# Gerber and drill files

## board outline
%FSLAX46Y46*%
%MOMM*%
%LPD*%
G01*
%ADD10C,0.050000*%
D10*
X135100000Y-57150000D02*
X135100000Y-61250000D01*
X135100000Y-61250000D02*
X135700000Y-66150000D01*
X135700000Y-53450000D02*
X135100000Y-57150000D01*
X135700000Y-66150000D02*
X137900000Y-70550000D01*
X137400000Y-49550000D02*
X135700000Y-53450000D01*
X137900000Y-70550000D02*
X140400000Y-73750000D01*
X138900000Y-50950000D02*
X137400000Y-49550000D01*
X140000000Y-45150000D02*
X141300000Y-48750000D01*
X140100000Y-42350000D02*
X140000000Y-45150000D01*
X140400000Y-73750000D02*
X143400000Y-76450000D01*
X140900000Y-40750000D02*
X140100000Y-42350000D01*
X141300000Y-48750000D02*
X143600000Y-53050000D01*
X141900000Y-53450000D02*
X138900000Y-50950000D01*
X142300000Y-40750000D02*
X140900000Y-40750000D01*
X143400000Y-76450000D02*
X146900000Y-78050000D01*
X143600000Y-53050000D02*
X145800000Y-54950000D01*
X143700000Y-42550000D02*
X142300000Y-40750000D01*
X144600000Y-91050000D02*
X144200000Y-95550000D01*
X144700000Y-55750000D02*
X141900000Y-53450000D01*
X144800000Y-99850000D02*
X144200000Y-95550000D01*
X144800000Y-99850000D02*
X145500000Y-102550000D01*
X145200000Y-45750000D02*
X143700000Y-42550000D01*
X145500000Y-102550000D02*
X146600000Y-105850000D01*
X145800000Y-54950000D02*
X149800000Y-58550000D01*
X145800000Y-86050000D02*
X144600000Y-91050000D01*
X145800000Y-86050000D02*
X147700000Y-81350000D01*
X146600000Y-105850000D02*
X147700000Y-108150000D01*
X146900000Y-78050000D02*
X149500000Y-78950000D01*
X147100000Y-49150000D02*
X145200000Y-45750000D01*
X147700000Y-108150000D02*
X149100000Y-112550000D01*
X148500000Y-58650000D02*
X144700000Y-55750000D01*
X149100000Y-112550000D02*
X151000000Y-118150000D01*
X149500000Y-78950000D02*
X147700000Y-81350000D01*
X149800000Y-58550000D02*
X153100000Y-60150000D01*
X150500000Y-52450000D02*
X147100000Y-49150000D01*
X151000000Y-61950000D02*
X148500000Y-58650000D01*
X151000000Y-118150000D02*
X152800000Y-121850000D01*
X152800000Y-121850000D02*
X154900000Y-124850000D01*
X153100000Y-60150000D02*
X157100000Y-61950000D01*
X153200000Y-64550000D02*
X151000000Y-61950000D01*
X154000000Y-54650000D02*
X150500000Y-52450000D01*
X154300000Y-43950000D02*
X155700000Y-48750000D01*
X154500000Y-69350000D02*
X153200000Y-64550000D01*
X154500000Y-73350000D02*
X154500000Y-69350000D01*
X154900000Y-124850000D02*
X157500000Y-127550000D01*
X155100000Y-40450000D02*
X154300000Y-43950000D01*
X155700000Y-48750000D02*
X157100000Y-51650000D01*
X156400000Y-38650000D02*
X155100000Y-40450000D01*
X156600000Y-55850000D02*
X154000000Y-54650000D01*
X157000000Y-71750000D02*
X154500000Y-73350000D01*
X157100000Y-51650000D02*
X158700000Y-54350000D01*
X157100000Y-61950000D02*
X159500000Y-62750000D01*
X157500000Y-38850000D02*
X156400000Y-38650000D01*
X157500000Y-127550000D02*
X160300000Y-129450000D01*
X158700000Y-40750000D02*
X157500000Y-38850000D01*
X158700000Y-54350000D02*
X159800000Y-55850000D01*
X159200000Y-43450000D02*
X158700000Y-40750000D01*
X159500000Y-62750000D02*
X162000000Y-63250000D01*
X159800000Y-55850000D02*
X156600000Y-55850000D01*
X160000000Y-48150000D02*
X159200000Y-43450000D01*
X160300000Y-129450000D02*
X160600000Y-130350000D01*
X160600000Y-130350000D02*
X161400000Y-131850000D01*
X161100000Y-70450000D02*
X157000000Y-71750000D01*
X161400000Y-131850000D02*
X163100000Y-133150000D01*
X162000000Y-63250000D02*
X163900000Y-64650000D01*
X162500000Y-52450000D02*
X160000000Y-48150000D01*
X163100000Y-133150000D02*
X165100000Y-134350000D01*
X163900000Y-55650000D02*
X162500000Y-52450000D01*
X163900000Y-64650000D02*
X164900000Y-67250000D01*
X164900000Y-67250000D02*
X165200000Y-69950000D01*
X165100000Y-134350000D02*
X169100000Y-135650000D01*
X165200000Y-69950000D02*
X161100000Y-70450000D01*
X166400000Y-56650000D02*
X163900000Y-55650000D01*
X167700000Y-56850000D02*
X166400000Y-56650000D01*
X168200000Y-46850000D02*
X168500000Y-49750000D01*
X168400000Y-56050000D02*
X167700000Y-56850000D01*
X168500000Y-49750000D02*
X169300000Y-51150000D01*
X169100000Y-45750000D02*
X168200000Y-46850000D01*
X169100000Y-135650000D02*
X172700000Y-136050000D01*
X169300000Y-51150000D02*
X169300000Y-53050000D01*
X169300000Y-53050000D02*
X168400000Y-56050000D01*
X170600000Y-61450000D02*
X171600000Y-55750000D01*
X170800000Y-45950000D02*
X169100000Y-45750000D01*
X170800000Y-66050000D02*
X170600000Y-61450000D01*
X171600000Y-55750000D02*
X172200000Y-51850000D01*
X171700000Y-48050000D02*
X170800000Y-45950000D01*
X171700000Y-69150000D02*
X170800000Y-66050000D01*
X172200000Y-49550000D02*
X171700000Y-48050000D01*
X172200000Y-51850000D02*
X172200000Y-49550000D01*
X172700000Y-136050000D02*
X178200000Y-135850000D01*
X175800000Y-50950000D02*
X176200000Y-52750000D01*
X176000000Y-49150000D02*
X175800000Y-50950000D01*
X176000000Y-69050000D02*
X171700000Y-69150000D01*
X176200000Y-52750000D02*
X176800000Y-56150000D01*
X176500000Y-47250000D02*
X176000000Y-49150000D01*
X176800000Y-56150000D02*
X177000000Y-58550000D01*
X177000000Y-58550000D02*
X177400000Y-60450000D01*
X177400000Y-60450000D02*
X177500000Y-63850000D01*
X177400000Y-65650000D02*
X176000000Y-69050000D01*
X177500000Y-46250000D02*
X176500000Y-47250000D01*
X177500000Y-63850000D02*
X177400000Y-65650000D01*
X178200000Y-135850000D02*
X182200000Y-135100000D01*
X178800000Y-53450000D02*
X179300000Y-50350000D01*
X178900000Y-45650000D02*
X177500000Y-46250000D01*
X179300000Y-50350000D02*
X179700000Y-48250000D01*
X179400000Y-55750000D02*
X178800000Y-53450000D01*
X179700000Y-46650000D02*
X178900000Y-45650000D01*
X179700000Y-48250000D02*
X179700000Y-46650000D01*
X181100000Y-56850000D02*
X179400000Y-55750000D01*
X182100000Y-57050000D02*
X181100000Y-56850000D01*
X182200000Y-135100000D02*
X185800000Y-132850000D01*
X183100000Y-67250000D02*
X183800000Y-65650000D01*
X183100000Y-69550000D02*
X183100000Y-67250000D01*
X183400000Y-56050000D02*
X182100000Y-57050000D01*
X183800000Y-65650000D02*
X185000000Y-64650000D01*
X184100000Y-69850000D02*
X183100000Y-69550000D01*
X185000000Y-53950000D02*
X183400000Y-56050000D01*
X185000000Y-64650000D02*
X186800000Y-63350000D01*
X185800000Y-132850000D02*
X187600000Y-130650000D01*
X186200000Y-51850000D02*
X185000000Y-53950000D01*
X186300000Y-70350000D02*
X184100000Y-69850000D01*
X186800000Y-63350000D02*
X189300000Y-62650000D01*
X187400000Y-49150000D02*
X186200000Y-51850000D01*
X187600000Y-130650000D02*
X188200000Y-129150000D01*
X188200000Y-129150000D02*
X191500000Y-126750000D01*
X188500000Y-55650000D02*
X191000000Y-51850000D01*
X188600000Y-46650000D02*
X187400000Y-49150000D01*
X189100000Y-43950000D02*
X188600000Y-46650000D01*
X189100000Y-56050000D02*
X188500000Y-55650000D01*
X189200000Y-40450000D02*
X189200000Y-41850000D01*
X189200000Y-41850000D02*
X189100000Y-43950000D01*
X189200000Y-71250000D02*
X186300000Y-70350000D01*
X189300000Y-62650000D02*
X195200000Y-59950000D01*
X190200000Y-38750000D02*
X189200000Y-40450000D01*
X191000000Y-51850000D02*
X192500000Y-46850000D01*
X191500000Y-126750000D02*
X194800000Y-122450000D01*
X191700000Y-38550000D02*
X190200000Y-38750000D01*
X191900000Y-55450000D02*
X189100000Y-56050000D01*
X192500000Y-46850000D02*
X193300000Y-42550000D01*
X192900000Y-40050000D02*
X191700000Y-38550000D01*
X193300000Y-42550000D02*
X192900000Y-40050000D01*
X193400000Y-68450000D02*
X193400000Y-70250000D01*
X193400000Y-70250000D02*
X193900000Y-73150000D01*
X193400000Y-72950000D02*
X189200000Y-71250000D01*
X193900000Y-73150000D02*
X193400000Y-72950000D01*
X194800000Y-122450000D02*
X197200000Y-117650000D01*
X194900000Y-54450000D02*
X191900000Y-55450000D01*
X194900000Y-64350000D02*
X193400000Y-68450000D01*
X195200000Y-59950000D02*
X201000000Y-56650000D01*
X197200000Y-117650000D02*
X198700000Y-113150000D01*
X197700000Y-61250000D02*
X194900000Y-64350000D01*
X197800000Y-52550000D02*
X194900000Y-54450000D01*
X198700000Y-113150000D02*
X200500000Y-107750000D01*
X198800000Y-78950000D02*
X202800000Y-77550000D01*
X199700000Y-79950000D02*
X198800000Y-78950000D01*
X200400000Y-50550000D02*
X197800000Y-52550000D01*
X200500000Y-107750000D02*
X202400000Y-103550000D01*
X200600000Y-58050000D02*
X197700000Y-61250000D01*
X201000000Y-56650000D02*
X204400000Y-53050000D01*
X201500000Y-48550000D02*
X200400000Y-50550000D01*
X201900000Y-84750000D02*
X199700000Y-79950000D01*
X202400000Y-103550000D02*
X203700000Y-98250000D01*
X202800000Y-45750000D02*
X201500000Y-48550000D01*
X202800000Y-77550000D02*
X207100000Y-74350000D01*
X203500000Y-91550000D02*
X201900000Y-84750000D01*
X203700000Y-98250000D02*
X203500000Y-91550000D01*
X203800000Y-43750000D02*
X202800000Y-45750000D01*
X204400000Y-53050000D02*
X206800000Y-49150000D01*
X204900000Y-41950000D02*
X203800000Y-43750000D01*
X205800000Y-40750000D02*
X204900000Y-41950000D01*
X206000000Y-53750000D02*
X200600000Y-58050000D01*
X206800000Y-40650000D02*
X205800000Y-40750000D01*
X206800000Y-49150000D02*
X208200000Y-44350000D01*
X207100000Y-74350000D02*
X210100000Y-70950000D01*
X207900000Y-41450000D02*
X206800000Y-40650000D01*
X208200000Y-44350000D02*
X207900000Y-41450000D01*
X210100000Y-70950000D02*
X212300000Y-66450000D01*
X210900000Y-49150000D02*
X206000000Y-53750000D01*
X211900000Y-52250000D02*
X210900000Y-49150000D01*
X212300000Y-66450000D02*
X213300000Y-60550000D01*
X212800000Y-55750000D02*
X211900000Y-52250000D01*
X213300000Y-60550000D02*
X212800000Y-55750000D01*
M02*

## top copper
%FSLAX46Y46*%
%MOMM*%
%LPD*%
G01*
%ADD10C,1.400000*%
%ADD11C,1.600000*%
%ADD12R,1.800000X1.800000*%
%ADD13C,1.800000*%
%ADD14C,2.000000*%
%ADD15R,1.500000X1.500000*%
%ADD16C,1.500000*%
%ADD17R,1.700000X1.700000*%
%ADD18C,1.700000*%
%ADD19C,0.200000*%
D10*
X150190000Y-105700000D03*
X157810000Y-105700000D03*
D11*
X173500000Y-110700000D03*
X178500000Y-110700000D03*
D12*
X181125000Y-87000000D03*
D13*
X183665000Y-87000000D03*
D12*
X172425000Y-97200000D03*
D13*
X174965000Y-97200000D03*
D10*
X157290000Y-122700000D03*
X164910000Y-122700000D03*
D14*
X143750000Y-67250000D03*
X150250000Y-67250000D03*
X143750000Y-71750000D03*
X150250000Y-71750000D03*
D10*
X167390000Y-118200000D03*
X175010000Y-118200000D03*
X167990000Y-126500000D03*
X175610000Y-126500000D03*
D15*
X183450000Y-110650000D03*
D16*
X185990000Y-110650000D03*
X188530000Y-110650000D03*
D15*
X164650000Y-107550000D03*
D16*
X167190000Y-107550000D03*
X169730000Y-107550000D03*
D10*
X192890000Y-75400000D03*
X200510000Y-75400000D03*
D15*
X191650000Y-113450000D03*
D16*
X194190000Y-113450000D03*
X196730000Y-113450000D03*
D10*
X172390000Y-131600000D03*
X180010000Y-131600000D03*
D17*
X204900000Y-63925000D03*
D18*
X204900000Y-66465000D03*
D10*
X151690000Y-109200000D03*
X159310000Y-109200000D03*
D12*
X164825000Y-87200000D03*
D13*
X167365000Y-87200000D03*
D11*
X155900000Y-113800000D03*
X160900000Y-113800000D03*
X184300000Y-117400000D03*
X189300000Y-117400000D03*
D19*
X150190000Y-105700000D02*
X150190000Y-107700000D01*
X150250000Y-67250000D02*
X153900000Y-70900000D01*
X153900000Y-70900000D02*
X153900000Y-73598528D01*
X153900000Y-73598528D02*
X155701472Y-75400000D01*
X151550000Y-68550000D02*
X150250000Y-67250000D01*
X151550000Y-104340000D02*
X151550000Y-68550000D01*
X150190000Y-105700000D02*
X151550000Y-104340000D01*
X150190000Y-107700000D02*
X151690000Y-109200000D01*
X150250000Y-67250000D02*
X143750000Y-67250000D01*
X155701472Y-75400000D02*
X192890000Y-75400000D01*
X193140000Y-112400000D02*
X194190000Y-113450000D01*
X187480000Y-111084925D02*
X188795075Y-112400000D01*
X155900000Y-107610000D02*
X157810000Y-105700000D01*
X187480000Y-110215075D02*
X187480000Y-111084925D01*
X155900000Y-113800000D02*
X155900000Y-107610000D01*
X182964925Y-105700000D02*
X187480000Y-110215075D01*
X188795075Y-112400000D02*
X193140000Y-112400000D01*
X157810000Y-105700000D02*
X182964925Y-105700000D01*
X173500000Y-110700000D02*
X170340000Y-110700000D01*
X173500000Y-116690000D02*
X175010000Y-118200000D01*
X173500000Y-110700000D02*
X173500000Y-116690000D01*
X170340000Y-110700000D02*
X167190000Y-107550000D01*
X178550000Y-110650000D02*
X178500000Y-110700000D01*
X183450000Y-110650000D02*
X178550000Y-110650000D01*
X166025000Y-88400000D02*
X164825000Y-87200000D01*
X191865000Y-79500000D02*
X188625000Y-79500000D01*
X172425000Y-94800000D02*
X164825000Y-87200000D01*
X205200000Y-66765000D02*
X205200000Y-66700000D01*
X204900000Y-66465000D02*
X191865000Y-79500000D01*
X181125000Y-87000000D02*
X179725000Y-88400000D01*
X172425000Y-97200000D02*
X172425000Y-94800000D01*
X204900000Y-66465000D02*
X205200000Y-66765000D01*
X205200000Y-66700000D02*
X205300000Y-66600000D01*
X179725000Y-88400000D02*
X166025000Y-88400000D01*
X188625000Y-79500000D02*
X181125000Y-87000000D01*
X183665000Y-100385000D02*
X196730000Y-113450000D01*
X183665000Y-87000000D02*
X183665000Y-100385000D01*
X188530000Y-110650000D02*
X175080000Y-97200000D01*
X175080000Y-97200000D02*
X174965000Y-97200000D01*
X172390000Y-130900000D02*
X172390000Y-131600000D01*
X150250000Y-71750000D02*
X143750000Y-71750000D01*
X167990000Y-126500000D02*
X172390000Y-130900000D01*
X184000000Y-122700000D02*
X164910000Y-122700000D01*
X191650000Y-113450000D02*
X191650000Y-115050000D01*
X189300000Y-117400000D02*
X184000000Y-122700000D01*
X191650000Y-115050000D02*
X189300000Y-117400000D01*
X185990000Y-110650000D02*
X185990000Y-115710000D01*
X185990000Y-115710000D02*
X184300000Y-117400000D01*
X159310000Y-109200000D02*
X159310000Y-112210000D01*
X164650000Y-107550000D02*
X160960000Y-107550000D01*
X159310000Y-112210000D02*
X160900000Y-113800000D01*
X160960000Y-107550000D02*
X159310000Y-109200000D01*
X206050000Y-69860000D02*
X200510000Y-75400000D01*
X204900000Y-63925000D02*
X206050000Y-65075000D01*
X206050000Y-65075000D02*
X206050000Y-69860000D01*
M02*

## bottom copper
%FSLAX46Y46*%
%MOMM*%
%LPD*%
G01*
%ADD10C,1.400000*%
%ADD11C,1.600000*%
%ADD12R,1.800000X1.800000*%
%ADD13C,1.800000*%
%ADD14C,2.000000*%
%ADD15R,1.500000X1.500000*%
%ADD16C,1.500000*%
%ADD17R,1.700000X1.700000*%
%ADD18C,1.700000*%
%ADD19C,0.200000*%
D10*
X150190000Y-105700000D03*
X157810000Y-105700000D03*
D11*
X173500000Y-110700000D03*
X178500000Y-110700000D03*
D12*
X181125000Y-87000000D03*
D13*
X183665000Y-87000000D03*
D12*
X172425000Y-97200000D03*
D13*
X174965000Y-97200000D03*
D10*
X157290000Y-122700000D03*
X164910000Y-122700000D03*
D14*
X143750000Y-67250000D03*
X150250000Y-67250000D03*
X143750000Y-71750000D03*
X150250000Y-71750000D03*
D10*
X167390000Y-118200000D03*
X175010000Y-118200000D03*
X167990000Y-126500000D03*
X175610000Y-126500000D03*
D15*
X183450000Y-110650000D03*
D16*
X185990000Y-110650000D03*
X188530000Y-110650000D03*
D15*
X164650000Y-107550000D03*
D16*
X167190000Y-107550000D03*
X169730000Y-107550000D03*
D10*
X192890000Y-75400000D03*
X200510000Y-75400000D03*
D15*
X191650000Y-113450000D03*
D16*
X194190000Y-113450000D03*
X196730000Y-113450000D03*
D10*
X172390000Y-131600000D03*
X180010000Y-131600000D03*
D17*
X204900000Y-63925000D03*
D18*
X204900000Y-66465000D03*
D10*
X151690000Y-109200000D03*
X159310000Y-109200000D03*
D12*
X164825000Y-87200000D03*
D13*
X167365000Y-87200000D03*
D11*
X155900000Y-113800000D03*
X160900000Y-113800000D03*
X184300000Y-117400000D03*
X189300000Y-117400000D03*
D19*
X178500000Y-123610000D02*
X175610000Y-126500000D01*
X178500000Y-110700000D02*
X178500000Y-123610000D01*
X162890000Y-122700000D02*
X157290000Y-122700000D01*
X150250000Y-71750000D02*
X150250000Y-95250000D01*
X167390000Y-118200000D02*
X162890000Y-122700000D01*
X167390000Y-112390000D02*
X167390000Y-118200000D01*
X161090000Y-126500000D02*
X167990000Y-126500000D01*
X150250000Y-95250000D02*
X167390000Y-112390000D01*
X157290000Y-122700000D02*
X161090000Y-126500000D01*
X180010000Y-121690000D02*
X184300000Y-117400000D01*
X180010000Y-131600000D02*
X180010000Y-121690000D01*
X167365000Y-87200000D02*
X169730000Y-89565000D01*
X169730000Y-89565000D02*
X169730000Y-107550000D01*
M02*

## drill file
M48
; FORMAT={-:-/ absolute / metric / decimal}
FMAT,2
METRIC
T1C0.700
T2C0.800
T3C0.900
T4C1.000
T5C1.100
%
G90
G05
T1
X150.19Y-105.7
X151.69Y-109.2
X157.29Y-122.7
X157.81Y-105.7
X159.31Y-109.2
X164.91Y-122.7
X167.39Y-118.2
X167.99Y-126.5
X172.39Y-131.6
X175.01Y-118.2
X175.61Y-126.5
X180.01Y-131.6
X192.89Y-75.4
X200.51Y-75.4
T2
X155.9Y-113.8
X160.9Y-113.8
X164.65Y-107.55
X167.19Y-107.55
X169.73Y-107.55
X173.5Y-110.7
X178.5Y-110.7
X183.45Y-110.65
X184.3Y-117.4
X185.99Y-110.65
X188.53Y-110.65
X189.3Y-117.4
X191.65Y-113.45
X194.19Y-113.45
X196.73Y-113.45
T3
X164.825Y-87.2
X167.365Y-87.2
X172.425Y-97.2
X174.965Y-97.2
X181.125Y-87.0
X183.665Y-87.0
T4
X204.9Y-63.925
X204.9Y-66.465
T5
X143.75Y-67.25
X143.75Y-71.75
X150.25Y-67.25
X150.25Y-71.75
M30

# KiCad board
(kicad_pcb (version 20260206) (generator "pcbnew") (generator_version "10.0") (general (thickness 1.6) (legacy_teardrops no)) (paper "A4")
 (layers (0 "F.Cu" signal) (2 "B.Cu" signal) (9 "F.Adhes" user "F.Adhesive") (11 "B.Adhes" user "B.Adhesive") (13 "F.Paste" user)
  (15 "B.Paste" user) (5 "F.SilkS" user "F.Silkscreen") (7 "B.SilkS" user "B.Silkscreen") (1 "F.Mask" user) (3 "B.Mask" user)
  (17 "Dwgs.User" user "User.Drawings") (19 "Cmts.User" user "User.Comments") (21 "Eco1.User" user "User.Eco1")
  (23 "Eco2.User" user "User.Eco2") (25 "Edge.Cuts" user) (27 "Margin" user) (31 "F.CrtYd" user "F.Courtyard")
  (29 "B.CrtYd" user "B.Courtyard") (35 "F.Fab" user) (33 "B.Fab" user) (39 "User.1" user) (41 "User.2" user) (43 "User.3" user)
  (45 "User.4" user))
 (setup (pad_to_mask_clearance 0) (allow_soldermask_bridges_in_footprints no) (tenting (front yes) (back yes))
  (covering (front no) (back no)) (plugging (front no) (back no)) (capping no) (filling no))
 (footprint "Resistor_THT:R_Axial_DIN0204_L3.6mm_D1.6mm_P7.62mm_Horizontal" (layer "F.Cu") (at 150.19 105.7)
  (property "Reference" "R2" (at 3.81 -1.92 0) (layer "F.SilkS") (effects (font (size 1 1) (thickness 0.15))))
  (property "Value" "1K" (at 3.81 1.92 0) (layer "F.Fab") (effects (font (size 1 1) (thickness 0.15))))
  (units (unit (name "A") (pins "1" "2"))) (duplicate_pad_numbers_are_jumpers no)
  (pad "1" thru_hole circle (at 0 0) (size 1.4 1.4) (drill 0.7) (layers "*.Cu" "*.Mask") (remove_unused_layers no) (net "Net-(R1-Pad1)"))
  (pad "2" thru_hole circle (at 7.62 0) (size 1.4 1.4) (drill 0.7) (layers "*.Cu" "*.Mask") (remove_unused_layers no) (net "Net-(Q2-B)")))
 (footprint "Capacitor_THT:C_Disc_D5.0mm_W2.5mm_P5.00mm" (layer "F.Cu") (at 173.5 110.7)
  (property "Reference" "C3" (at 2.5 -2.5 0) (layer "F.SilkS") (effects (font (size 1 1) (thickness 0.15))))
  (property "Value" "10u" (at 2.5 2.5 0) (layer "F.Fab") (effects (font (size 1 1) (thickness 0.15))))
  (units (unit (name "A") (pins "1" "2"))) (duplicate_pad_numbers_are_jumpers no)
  (pad "1" thru_hole circle (at 0 0) (size 1.6 1.6) (drill 0.8) (layers "*.Cu" "*.Mask") (remove_unused_layers no) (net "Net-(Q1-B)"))
  (pad "2" thru_hole circle (at 5 0) (size 1.6 1.6) (drill 0.8) (layers "*.Cu" "*.Mask") (remove_unused_layers no) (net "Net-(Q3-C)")))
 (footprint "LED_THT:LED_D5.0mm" (layer "F.Cu") (at 181.125 87)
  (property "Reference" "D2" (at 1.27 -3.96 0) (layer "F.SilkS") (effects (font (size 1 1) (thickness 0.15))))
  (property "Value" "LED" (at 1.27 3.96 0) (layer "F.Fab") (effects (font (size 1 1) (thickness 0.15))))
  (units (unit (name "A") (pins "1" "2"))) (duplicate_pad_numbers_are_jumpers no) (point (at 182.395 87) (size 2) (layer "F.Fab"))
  (pad "1" thru_hole rect (at 0 0) (size 1.8 1.8) (drill 0.9) (layers "*.Cu" "*.Mask") (remove_unused_layers no) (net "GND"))
  (pad "2" thru_hole circle (at 2.54 0) (size 1.8 1.8) (drill 0.9) (layers "*.Cu" "*.Mask") (remove_unused_layers no) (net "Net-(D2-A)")))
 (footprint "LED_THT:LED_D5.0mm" (layer "F.Cu") (at 172.425 97.2)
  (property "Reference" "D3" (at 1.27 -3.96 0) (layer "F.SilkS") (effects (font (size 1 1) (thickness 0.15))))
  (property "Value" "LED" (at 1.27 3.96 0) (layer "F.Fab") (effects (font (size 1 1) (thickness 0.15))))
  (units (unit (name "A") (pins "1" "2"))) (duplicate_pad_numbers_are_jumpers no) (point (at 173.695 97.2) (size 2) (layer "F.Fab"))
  (pad "1" thru_hole rect (at 0 0) (size 1.8 1.8) (drill 0.9) (layers "*.Cu" "*.Mask") (remove_unused_layers no) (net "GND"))
  (pad "2" thru_hole circle (at 2.54 0) (size 1.8 1.8) (drill 0.9) (layers "*.Cu" "*.Mask") (remove_unused_layers no) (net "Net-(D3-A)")))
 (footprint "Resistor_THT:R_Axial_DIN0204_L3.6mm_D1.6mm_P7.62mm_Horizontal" (layer "F.Cu") (at 157.29 122.7)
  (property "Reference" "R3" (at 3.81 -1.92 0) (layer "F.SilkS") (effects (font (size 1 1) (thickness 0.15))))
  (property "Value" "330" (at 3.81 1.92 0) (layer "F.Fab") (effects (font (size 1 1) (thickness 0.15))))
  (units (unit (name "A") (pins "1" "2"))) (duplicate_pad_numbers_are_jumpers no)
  (pad "1" thru_hole circle (at 0 0) (size 1.4 1.4) (drill 0.7) (layers "*.Cu" "*.Mask") (remove_unused_layers no) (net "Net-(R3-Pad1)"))
  (pad "2" thru_hole circle (at 7.62 0) (size 1.4 1.4) (drill 0.7) (layers "*.Cu" "*.Mask") (remove_unused_layers no) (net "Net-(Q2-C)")))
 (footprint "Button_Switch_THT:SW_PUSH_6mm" (layer "F.Cu") (at 143.75 67.25)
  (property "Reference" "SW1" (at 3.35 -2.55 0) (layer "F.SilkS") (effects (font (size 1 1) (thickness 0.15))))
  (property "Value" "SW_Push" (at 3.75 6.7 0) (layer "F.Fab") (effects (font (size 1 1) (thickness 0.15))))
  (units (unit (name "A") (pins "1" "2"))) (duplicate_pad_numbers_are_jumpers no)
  (pad "1" thru_hole circle (at 0 0 90) (size 2 2) (drill 1.1) (layers "*.Cu" "*.Mask") (remove_unused_layers no) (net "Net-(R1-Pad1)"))
  (pad "1" thru_hole circle (at 6.5 0 90) (size 2 2) (drill 1.1) (layers "*.Cu" "*.Mask") (remove_unused_layers no) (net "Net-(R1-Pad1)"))
  (pad "2" thru_hole circle (at 0 4.5 90) (size 2 2) (drill 1.1) (layers "*.Cu" "*.Mask") (remove_unused_layers no) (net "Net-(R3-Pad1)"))
  (pad "2" thru_hole circle (at 6.5 4.5 90) (size 2 2) (drill 1.1) (layers "*.Cu" "*.Mask") (remove_unused_layers no) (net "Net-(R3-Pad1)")))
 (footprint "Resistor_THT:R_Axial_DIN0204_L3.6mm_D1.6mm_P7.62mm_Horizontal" (layer "F.Cu") (at 167.39 118.2)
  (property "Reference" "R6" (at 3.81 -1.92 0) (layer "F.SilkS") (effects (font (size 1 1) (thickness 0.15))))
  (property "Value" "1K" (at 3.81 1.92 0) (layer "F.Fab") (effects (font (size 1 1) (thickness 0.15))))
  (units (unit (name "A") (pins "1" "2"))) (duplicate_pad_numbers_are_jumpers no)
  (pad "1" thru_hole circle (at 0 0) (size 1.4 1.4) (drill 0.7) (layers "*.Cu" "*.Mask") (remove_unused_layers no) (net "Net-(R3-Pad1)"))
  (pad "2" thru_hole circle (at 7.62 0) (size 1.4 1.4) (drill 0.7) (layers "*.Cu" "*.Mask") (remove_unused_layers no) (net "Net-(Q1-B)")))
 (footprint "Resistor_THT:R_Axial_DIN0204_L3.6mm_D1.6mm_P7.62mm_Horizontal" (layer "F.Cu") (at 167.99 126.5)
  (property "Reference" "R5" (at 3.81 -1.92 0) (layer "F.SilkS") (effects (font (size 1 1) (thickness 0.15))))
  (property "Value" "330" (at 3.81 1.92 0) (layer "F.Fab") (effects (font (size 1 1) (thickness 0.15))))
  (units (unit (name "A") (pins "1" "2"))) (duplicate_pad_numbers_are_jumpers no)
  (pad "1" thru_hole circle (at 0 0) (size 1.4 1.4) (drill 0.7) (layers "*.Cu" "*.Mask") (remove_unused_layers no) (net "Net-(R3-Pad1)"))
  (pad "2" thru_hole circle (at 7.62 0) (size 1.4 1.4) (drill 0.7) (layers "*.Cu" "*.Mask") (remove_unused_layers no) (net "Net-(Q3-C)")))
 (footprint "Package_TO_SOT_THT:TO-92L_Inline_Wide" (layer "F.Cu") (at 183.45 110.65)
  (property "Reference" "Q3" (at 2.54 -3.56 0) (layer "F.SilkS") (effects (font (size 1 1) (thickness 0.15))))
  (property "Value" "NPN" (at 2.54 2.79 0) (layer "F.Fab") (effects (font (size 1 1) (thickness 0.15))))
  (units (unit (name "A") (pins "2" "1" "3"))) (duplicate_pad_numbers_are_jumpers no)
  (pad "1" thru_hole rect (at 0 0) (size 1.5 1.5) (drill 0.8) (layers "*.Cu" "*.Mask") (remove_unused_layers no) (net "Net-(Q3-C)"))
  (pad "2" thru_hole circle (at 2.54 0) (size 1.5 1.5) (drill 0.8) (layers "*.Cu" "*.Mask") (remove_unused_layers no) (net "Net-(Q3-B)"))
  (pad "3" thru_hole circle (at 5.08 0) (size 1.5 1.5) (drill 0.8) (layers "*.Cu" "*.Mask") (remove_unused_layers no) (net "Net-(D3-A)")))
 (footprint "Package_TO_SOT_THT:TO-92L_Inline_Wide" (layer "F.Cu") (at 164.65 107.55)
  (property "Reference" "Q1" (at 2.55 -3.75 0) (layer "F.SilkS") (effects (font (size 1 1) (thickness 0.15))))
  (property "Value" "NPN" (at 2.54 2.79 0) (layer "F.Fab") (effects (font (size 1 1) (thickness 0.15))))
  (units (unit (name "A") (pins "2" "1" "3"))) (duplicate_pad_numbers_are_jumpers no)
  (pad "1" thru_hole rect (at 0 0) (size 1.5 1.5) (drill 0.8) (layers "*.Cu" "*.Mask") (remove_unused_layers no) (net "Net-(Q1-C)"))
  (pad "2" thru_hole circle (at 2.54 0) (size 1.5 1.5) (drill 0.8) (layers "*.Cu" "*.Mask") (remove_unused_layers no) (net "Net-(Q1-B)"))
  (pad "3" thru_hole circle (at 5.08 0) (size 1.5 1.5) (drill 0.8) (layers "*.Cu" "*.Mask") (remove_unused_layers no) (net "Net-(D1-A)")))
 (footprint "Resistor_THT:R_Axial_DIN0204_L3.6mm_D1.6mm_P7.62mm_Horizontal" (layer "F.Cu") (at 192.89 75.4)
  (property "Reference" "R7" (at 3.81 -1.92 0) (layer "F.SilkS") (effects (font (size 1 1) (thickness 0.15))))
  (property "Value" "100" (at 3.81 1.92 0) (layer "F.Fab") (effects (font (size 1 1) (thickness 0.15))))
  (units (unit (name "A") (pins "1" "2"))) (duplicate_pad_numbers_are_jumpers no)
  (pad "1" thru_hole circle (at 0 0) (size 1.4 1.4) (drill 0.7) (layers "*.Cu" "*.Mask") (remove_unused_layers no) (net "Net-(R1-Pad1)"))
  (pad "2" thru_hole circle (at 7.62 0) (size 1.4 1.4) (drill 0.7) (layers "*.Cu" "*.Mask") (remove_unused_layers no) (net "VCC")))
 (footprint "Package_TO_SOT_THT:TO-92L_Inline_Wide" (layer "F.Cu") (at 191.65 113.45)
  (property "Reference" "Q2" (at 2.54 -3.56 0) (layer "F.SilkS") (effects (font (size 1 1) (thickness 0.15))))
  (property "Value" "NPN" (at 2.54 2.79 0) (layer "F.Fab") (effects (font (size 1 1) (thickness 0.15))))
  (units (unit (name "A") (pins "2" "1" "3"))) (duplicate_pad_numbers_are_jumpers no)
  (pad "1" thru_hole rect (at 0 0) (size 1.5 1.5) (drill 0.8) (layers "*.Cu" "*.Mask") (remove_unused_layers no) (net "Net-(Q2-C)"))
  (pad "2" thru_hole circle (at 2.54 0) (size 1.5 1.5) (drill 0.8) (layers "*.Cu" "*.Mask") (remove_unused_layers no) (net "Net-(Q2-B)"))
  (pad "3" thru_hole circle (at 5.08 0) (size 1.5 1.5) (drill 0.8) (layers "*.Cu" "*.Mask") (remove_unused_layers no) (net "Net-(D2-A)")))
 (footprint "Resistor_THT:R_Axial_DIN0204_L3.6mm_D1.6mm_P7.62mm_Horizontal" (layer "F.Cu") (at 172.39 131.6)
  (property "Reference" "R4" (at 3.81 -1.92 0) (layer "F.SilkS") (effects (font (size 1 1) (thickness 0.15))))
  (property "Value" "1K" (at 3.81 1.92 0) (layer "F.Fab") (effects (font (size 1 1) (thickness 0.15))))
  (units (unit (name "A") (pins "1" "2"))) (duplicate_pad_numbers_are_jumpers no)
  (pad "1" thru_hole circle (at 0 0) (size 1.4 1.4) (drill 0.7) (layers "*.Cu" "*.Mask") (remove_unused_layers no) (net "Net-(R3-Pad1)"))
  (pad "2" thru_hole circle (at 7.62 0) (size 1.4 1.4) (drill 0.7) (layers "*.Cu" "*.Mask") (remove_unused_layers no) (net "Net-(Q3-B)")))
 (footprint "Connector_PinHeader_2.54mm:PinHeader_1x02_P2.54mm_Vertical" (layer "F.Cu") (at 204.9 63.925)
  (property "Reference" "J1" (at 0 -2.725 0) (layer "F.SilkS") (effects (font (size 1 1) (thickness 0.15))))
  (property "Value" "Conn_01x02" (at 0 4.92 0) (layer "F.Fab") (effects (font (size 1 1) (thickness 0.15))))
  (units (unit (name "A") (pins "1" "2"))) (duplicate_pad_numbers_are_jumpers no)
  (pad "1" thru_hole rect (at 0 0) (size 1.7 1.7) (drill 1) (layers "*.Cu" "*.Mask") (remove_unused_layers no) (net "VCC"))
  (pad "2" thru_hole circle (at 0 2.54) (size 1.7 1.7) (drill 1) (layers "*.Cu" "*.Mask") (remove_unused_layers no) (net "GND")))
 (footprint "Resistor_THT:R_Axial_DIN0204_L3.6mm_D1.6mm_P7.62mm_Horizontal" (layer "F.Cu") (at 151.69 109.2)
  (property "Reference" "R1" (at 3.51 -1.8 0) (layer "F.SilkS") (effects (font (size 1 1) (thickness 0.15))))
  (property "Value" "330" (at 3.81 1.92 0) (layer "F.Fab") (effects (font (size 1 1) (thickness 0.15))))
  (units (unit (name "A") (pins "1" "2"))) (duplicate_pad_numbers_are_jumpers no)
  (pad "1" thru_hole circle (at 0 0) (size 1.4 1.4) (drill 0.7) (layers "*.Cu" "*.Mask") (remove_unused_layers no) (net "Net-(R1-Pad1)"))
  (pad "2" thru_hole circle (at 7.62 0) (size 1.4 1.4) (drill 0.7) (layers "*.Cu" "*.Mask") (remove_unused_layers no) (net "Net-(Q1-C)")))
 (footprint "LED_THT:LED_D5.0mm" (layer "F.Cu") (at 164.825 87.2)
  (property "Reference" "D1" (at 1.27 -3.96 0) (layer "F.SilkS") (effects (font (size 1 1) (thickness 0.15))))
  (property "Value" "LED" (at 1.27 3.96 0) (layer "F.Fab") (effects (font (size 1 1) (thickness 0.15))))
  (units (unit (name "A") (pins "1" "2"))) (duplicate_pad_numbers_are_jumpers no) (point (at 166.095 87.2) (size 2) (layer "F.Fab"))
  (pad "1" thru_hole rect (at 0 0) (size 1.8 1.8) (drill 0.9) (layers "*.Cu" "*.Mask") (remove_unused_layers no) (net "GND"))
  (pad "2" thru_hole circle (at 2.54 0) (size 1.8 1.8) (drill 0.9) (layers "*.Cu" "*.Mask") (remove_unused_layers no) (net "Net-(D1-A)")))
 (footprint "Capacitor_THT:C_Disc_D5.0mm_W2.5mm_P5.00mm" (layer "F.Cu") (at 155.9 113.8)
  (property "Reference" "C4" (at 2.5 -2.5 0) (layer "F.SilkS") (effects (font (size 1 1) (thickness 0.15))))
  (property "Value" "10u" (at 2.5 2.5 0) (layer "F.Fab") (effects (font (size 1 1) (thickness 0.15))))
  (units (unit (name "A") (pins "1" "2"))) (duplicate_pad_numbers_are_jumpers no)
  (pad "1" thru_hole circle (at 0 0) (size 1.6 1.6) (drill 0.8) (layers "*.Cu" "*.Mask") (remove_unused_layers no) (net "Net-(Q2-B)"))
  (pad "2" thru_hole circle (at 5 0) (size 1.6 1.6) (drill 0.8) (layers "*.Cu" "*.Mask") (remove_unused_layers no) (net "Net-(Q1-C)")))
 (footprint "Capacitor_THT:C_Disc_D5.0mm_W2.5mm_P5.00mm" (layer "F.Cu") (at 184.3 117.4)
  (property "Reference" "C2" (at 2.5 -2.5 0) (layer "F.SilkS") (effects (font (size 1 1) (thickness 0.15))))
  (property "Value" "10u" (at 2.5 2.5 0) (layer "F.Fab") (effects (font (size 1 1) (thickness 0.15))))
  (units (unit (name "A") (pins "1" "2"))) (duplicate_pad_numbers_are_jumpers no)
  (pad "1" thru_hole circle (at 0 0) (size 1.6 1.6) (drill 0.8) (layers "*.Cu" "*.Mask") (remove_unused_layers no) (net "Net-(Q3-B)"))
  (pad "2" thru_hole circle (at 5 0) (size 1.6 1.6) (drill 0.8) (layers "*.Cu" "*.Mask") (remove_unused_layers no) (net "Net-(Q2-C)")))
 (gr_line (start 135.1 57.15) (end 135.1 61.25) (stroke (width 0.05) (type default)) (layer "Edge.Cuts"))
 (gr_line (start 135.1 61.25) (end 135.7 66.15) (stroke (width 0.05) (type default)) (layer "Edge.Cuts"))
 (gr_line (start 135.7 53.45) (end 135.1 57.15) (stroke (width 0.05) (type default)) (layer "Edge.Cuts"))
 (gr_line (start 135.7 66.15) (end 137.9 70.55) (stroke (width 0.05) (type default)) (layer "Edge.Cuts"))
 (gr_line (start 137.4 49.55) (end 135.7 53.45) (stroke (width 0.05) (type default)) (layer "Edge.Cuts"))
 (gr_line (start 137.9 70.55) (end 140.4 73.75) (stroke (width 0.05) (type default)) (layer "Edge.Cuts"))
 (gr_line (start 138.9 50.95) (end 137.4 49.55) (stroke (width 0.05) (type default)) (layer "Edge.Cuts"))
 (gr_line (start 140 45.15) (end 141.3 48.75) (stroke (width 0.05) (type default)) (layer "Edge.Cuts"))
 (gr_line (start 140.1 42.35) (end 140 45.15) (stroke (width 0.05) (type default)) (layer "Edge.Cuts"))
 (gr_line (start 140.4 73.75) (end 143.4 76.45) (stroke (width 0.05) (type default)) (layer "Edge.Cuts"))
 (gr_line (start 140.9 40.75) (end 140.1 42.35) (stroke (width 0.05) (type default)) (layer "Edge.Cuts"))
 (gr_line (start 141.3 48.75) (end 143.6 53.05) (stroke (width 0.05) (type default)) (layer "Edge.Cuts"))
 (gr_line (start 141.9 53.45) (end 138.9 50.95) (stroke (width 0.05) (type default)) (layer "Edge.Cuts"))
 (gr_line (start 142.3 40.75) (end 140.9 40.75) (stroke (width 0.05) (type default)) (layer "Edge.Cuts"))
 (gr_line (start 143.4 76.45) (end 146.9 78.05) (stroke (width 0.05) (type default)) (layer "Edge.Cuts"))
 (gr_line (start 143.6 53.05) (end 145.8 54.95) (stroke (width 0.05) (type default)) (layer "Edge.Cuts"))
 (gr_line (start 143.7 42.55) (end 142.3 40.75) (stroke (width 0.05) (type default)) (layer "Edge.Cuts"))
 (gr_line (start 144.6 91.05) (end 144.2 95.55) (stroke (width 0.05) (type default)) (layer "Edge.Cuts"))
 (gr_line (start 144.7 55.75) (end 141.9 53.45) (stroke (width 0.05) (type default)) (layer "Edge.Cuts"))
 (gr_line (start 144.8 99.85) (end 144.2 95.55) (stroke (width 0.05) (type default)) (layer "Edge.Cuts"))
 (gr_line (start 144.8 99.85) (end 145.5 102.55) (stroke (width 0.05) (type default)) (layer "Edge.Cuts"))
 (gr_line (start 145.2 45.75) (end 143.7 42.55) (stroke (width 0.05) (type default)) (layer "Edge.Cuts"))
 (gr_line (start 145.5 102.55) (end 146.6 105.85) (stroke (width 0.05) (type default)) (layer "Edge.Cuts"))
 (gr_line (start 145.8 54.95) (end 149.8 58.55) (stroke (width 0.05) (type default)) (layer "Edge.Cuts"))
 (gr_line (start 145.8 86.05) (end 144.6 91.05) (stroke (width 0.05) (type default)) (layer "Edge.Cuts"))
 (gr_line (start 145.8 86.05) (end 147.7 81.35) (stroke (width 0.05) (type default)) (layer "Edge.Cuts"))
 (gr_line (start 146.6 105.85) (end 147.7 108.15) (stroke (width 0.05) (type default)) (layer "Edge.Cuts"))
 (gr_line (start 146.9 78.05) (end 149.5 78.95) (stroke (width 0.05) (type default)) (layer "Edge.Cuts"))
 (gr_line (start 147.1 49.15) (end 145.2 45.75) (stroke (width 0.05) (type default)) (layer "Edge.Cuts"))
 (gr_line (start 147.7 108.15) (end 149.1 112.55) (stroke (width 0.05) (type default)) (layer "Edge.Cuts"))
 (gr_line (start 148.5 58.65) (end 144.7 55.75) (stroke (width 0.05) (type default)) (layer "Edge.Cuts"))
 (gr_line (start 149.1 112.55) (end 151 118.15) (stroke (width 0.05) (type default)) (layer "Edge.Cuts"))
 (gr_line (start 149.5 78.95) (end 147.7 81.35) (stroke (width 0.05) (type default)) (layer "Edge.Cuts"))
 (gr_line (start 149.8 58.55) (end 153.1 60.15) (stroke (width 0.05) (type default)) (layer "Edge.Cuts"))
 (gr_line (start 150.5 52.45) (end 147.1 49.15) (stroke (width 0.05) (type default)) (layer "Edge.Cuts"))
 (gr_line (start 151 61.95) (end 148.5 58.65) (stroke (width 0.05) (type default)) (layer "Edge.Cuts"))
 (gr_line (start 151 118.15) (end 152.8 121.85) (stroke (width 0.05) (type default)) (layer "Edge.Cuts"))
 (gr_line (start 152.8 121.85) (end 154.9 124.85) (stroke (width 0.05) (type default)) (layer "Edge.Cuts"))
 (gr_line (start 153.1 60.15) (end 157.1 61.95) (stroke (width 0.05) (type default)) (layer "Edge.Cuts"))
 (gr_line (start 153.2 64.55) (end 151 61.95) (stroke (width 0.05) (type default)) (layer "Edge.Cuts"))
 (gr_line (start 154 54.65) (end 150.5 52.45) (stroke (width 0.05) (type default)) (layer "Edge.Cuts"))
 (gr_line (start 154.3 43.95) (end 155.7 48.75) (stroke (width 0.05) (type default)) (layer "Edge.Cuts"))
 (gr_line (start 154.5 69.35) (end 153.2 64.55) (stroke (width 0.05) (type default)) (layer "Edge.Cuts"))
 (gr_line (start 154.5 73.35) (end 154.5 69.35) (stroke (width 0.05) (type default)) (layer "Edge.Cuts"))
 (gr_line (start 154.9 124.85) (end 157.5 127.55) (stroke (width 0.05) (type default)) (layer "Edge.Cuts"))
 (gr_line (start 155.1 40.45) (end 154.3 43.95) (stroke (width 0.05) (type default)) (layer "Edge.Cuts"))
 (gr_line (start 155.7 48.75) (end 157.1 51.65) (stroke (width 0.05) (type default)) (layer "Edge.Cuts"))
 (gr_line (start 156.4 38.65) (end 155.1 40.45) (stroke (width 0.05) (type default)) (layer "Edge.Cuts"))
 (gr_line (start 156.6 55.85) (end 154 54.65) (stroke (width 0.05) (type default)) (layer "Edge.Cuts"))
 (gr_line (start 157 71.75) (end 154.5 73.35) (stroke (width 0.05) (type default)) (layer "Edge.Cuts"))
 (gr_line (start 157.1 51.65) (end 158.7 54.35) (stroke (width 0.05) (type default)) (layer "Edge.Cuts"))
 (gr_line (start 157.1 61.95) (end 159.5 62.75) (stroke (width 0.05) (type default)) (layer "Edge.Cuts"))
 (gr_line (start 157.5 38.85) (end 156.4 38.65) (stroke (width 0.05) (type default)) (layer "Edge.Cuts"))
 (gr_line (start 157.5 127.55) (end 160.3 129.45) (stroke (width 0.05) (type default)) (layer "Edge.Cuts"))
 (gr_line (start 158.7 40.75) (end 157.5 38.85) (stroke (width 0.05) (type default)) (layer "Edge.Cuts"))
 (gr_line (start 158.7 54.35) (end 159.8 55.85) (stroke (width 0.05) (type default)) (layer "Edge.Cuts"))
 (gr_line (start 159.2 43.45) (end 158.7 40.75) (stroke (width 0.05) (type default)) (layer "Edge.Cuts"))
 (gr_line (start 159.5 62.75) (end 162 63.25) (stroke (width 0.05) (type default)) (layer "Edge.Cuts"))
 (gr_line (start 159.8 55.85) (end 156.6 55.85) (stroke (width 0.05) (type default)) (layer "Edge.Cuts"))
 (gr_line (start 160 48.15) (end 159.2 43.45) (stroke (width 0.05) (type default)) (layer "Edge.Cuts"))
 (gr_line (start 160.3 129.45) (end 160.6 130.35) (stroke (width 0.05) (type default)) (layer "Edge.Cuts"))
 (gr_line (start 160.6 130.35) (end 161.4 131.85) (stroke (width 0.05) (type default)) (layer "Edge.Cuts"))
 (gr_line (start 161.1 70.45) (end 157 71.75) (stroke (width 0.05) (type default)) (layer "Edge.Cuts"))
 (gr_line (start 161.4 131.85) (end 163.1 133.15) (stroke (width 0.05) (type default)) (layer "Edge.Cuts"))
 (gr_line (start 162 63.25) (end 163.9 64.65) (stroke (width 0.05) (type default)) (layer "Edge.Cuts"))
 (gr_line (start 162.5 52.45) (end 160 48.15) (stroke (width 0.05) (type default)) (layer "Edge.Cuts"))
 (gr_line (start 163.1 133.15) (end 165.1 134.35) (stroke (width 0.05) (type default)) (layer "Edge.Cuts"))
 (gr_line (start 163.9 55.65) (end 162.5 52.45) (stroke (width 0.05) (type default)) (layer "Edge.Cuts"))
 (gr_line (start 163.9 64.65) (end 164.9 67.25) (stroke (width 0.05) (type default)) (layer "Edge.Cuts"))
 (gr_line (start 164.9 67.25) (end 165.2 69.95) (stroke (width 0.05) (type default)) (layer "Edge.Cuts"))
 (gr_line (start 165.1 134.35) (end 169.1 135.65) (stroke (width 0.05) (type default)) (layer "Edge.Cuts"))
 (gr_line (start 165.2 69.95) (end 161.1 70.45) (stroke (width 0.05) (type default)) (layer "Edge.Cuts"))
 (gr_line (start 166.4 56.65) (end 163.9 55.65) (stroke (width 0.05) (type default)) (layer "Edge.Cuts"))
 (gr_line (start 167.7 56.85) (end 166.4 56.65) (stroke (width 0.05) (type default)) (layer "Edge.Cuts"))
 (gr_line (start 168.2 46.85) (end 168.5 49.75) (stroke (width 0.05) (type default)) (layer "Edge.Cuts"))
 (gr_line (start 168.4 56.05) (end 167.7 56.85) (stroke (width 0.05) (type default)) (layer "Edge.Cuts"))
 (gr_line (start 168.5 49.75) (end 169.3 51.15) (stroke (width 0.05) (type default)) (layer "Edge.Cuts"))
 (gr_line (start 169.1 45.75) (end 168.2 46.85) (stroke (width 0.05) (type default)) (layer "Edge.Cuts"))
 (gr_line (start 169.1 135.65) (end 172.7 136.05) (stroke (width 0.05) (type default)) (layer "Edge.Cuts"))
 (gr_line (start 169.3 51.15) (end 169.3 53.05) (stroke (width 0.05) (type default)) (layer "Edge.Cuts"))
 (gr_line (start 169.3 53.05) (end 168.4 56.05) (stroke (width 0.05) (type default)) (layer "Edge.Cuts"))
 (gr_line (start 170.6 61.45) (end 171.6 55.75) (stroke (width 0.05) (type default)) (layer "Edge.Cuts"))
 (gr_line (start 170.8 45.95) (end 169.1 45.75) (stroke (width 0.05) (type default)) (layer "Edge.Cuts"))
 (gr_line (start 170.8 66.05) (end 170.6 61.45) (stroke (width 0.05) (type default)) (layer "Edge.Cuts"))
 (gr_line (start 171.6 55.75) (end 172.2 51.85) (stroke (width 0.05) (type default)) (layer "Edge.Cuts"))
 (gr_line (start 171.7 48.05) (end 170.8 45.95) (stroke (width 0.05) (type default)) (layer "Edge.Cuts"))
 (gr_line (start 171.7 69.15) (end 170.8 66.05) (stroke (width 0.05) (type default)) (layer "Edge.Cuts"))
 (gr_line (start 172.2 49.55) (end 171.7 48.05) (stroke (width 0.05) (type default)) (layer "Edge.Cuts"))
 (gr_line (start 172.2 51.85) (end 172.2 49.55) (stroke (width 0.05) (type default)) (layer "Edge.Cuts"))
 (gr_line (start 172.7 136.05) (end 178.2 135.85) (stroke (width 0.05) (type default)) (layer "Edge.Cuts"))
 (gr_line (start 175.8 50.95) (end 176.2 52.75) (stroke (width 0.05) (type default)) (layer "Edge.Cuts"))
 (gr_line (start 176 49.15) (end 175.8 50.95) (stroke (width 0.05) (type default)) (layer "Edge.Cuts"))
 (gr_line (start 176 69.05) (end 171.7 69.15) (stroke (width 0.05) (type default)) (layer "Edge.Cuts"))
 (gr_line (start 176.2 52.75) (end 176.8 56.15) (stroke (width 0.05) (type default)) (layer "Edge.Cuts"))
 (gr_line (start 176.5 47.25) (end 176 49.15) (stroke (width 0.05) (type default)) (layer "Edge.Cuts"))
 (gr_line (start 176.8 56.15) (end 177 58.55) (stroke (width 0.05) (type default)) (layer "Edge.Cuts"))
 (gr_line (start 177 58.55) (end 177.4 60.45) (stroke (width 0.05) (type default)) (layer "Edge.Cuts"))
 (gr_line (start 177.4 60.45) (end 177.5 63.85) (stroke (width 0.05) (type default)) (layer "Edge.Cuts"))
 (gr_line (start 177.4 65.65) (end 176 69.05) (stroke (width 0.05) (type default)) (layer "Edge.Cuts"))
 (gr_line (start 177.5 46.25) (end 176.5 47.25) (stroke (width 0.05) (type default)) (layer "Edge.Cuts"))
 (gr_line (start 177.5 63.85) (end 177.4 65.65) (stroke (width 0.05) (type default)) (layer "Edge.Cuts"))
 (gr_line (start 178.2 135.85) (end 182.2 135.1) (stroke (width 0.05) (type default)) (layer "Edge.Cuts"))
 (gr_line (start 178.8 53.45) (end 179.3 50.35) (stroke (width 0.05) (type default)) (layer "Edge.Cuts"))
 (gr_line (start 178.9 45.65) (end 177.5 46.25) (stroke (width 0.05) (type default)) (layer "Edge.Cuts"))
 (gr_line (start 179.3 50.35) (end 179.7 48.25) (stroke (width 0.05) (type default)) (layer "Edge.Cuts"))
 (gr_line (start 179.4 55.75) (end 178.8 53.45) (stroke (width 0.05) (type default)) (layer "Edge.Cuts"))
 (gr_line (start 179.7 46.65) (end 178.9 45.65) (stroke (width 0.05) (type default)) (layer "Edge.Cuts"))
 (gr_line (start 179.7 48.25) (end 179.7 46.65) (stroke (width 0.05) (type default)) (layer "Edge.Cuts"))
 (gr_line (start 181.1 56.85) (end 179.4 55.75) (stroke (width 0.05) (type default)) (layer "Edge.Cuts"))
 (gr_line (start 182.1 57.05) (end 181.1 56.85) (stroke (width 0.05) (type default)) (layer "Edge.Cuts"))
 (gr_line (start 182.2 135.1) (end 185.8 132.85) (stroke (width 0.05) (type default)) (layer "Edge.Cuts"))
 (gr_line (start 183.1 67.25) (end 183.8 65.65) (stroke (width 0.05) (type default)) (layer "Edge.Cuts"))
 (gr_line (start 183.1 69.55) (end 183.1 67.25) (stroke (width 0.05) (type default)) (layer "Edge.Cuts"))
 (gr_line (start 183.4 56.05) (end 182.1 57.05) (stroke (width 0.05) (type default)) (layer "Edge.Cuts"))
 (gr_line (start 183.8 65.65) (end 185 64.65) (stroke (width 0.05) (type default)) (layer "Edge.Cuts"))
 (gr_line (start 184.1 69.85) (end 183.1 69.55) (stroke (width 0.05) (type default)) (layer "Edge.Cuts"))
 (gr_line (start 185 53.95) (end 183.4 56.05) (stroke (width 0.05) (type default)) (layer "Edge.Cuts"))
 (gr_line (start 185 64.65) (end 186.8 63.35) (stroke (width 0.05) (type default)) (layer "Edge.Cuts"))
 (gr_line (start 185.8 132.85) (end 187.6 130.65) (stroke (width 0.05) (type default)) (layer "Edge.Cuts"))
 (gr_line (start 186.2 51.85) (end 185 53.95) (stroke (width 0.05) (type default)) (layer "Edge.Cuts"))
 (gr_line (start 186.3 70.35) (end 184.1 69.85) (stroke (width 0.05) (type default)) (layer "Edge.Cuts"))
 (gr_line (start 186.8 63.35) (end 189.3 62.65) (stroke (width 0.05) (type default)) (layer "Edge.Cuts"))
 (gr_line (start 187.4 49.15) (end 186.2 51.85) (stroke (width 0.05) (type default)) (layer "Edge.Cuts"))
 (gr_line (start 187.6 130.65) (end 188.2 129.15) (stroke (width 0.05) (type default)) (layer "Edge.Cuts"))
 (gr_line (start 188.2 129.15) (end 191.5 126.75) (stroke (width 0.05) (type default)) (layer "Edge.Cuts"))
 (gr_line (start 188.5 55.65) (end 191 51.85) (stroke (width 0.05) (type default)) (layer "Edge.Cuts"))
 (gr_line (start 188.6 46.65) (end 187.4 49.15) (stroke (width 0.05) (type default)) (layer "Edge.Cuts"))
 (gr_line (start 189.1 43.95) (end 188.6 46.65) (stroke (width 0.05) (type default)) (layer "Edge.Cuts"))
 (gr_line (start 189.1 56.05) (end 188.5 55.65) (stroke (width 0.05) (type default)) (layer "Edge.Cuts"))
 (gr_line (start 189.2 40.45) (end 189.2 41.85) (stroke (width 0.05) (type default)) (layer "Edge.Cuts"))
 (gr_line (start 189.2 41.85) (end 189.1 43.95) (stroke (width 0.05) (type default)) (layer "Edge.Cuts"))
 (gr_line (start 189.2 71.25) (end 186.3 70.35) (stroke (width 0.05) (type default)) (layer "Edge.Cuts"))
 (gr_line (start 189.3 62.65) (end 195.2 59.95) (stroke (width 0.05) (type default)) (layer "Edge.Cuts"))
 (gr_line (start 190.2 38.75) (end 189.2 40.45) (stroke (width 0.05) (type default)) (layer "Edge.Cuts"))
 (gr_line (start 191 51.85) (end 192.5 46.85) (stroke (width 0.05) (type default)) (layer "Edge.Cuts"))
 (gr_line (start 191.5 126.75) (end 194.8 122.45) (stroke (width 0.05) (type default)) (layer "Edge.Cuts"))
 (gr_line (start 191.7 38.55) (end 190.2 38.75) (stroke (width 0.05) (type default)) (layer "Edge.Cuts"))
 (gr_line (start 191.9 55.45) (end 189.1 56.05) (stroke (width 0.05) (type default)) (layer "Edge.Cuts"))
 (gr_line (start 192.5 46.85) (end 193.3 42.55) (stroke (width 0.05) (type default)) (layer "Edge.Cuts"))
 (gr_line (start 192.9 40.05) (end 191.7 38.55) (stroke (width 0.05) (type default)) (layer "Edge.Cuts"))
 (gr_line (start 193.3 42.55) (end 192.9 40.05) (stroke (width 0.05) (type default)) (layer "Edge.Cuts"))
 (gr_line (start 193.4 68.45) (end 193.4 70.25) (stroke (width 0.05) (type default)) (layer "Edge.Cuts"))
 (gr_line (start 193.4 70.25) (end 193.9 73.15) (stroke (width 0.05) (type default)) (layer "Edge.Cuts"))
 (gr_line (start 193.4 72.95) (end 189.2 71.25) (stroke (width 0.05) (type default)) (layer "Edge.Cuts"))
 (gr_line (start 193.9 73.15) (end 193.4 72.95) (stroke (width 0.05) (type default)) (layer "Edge.Cuts"))
 (gr_line (start 194.8 122.45) (end 197.2 117.65) (stroke (width 0.05) (type default)) (layer "Edge.Cuts"))
 (gr_line (start 194.9 54.45) (end 191.9 55.45) (stroke (width 0.05) (type default)) (layer "Edge.Cuts"))
 (gr_line (start 194.9 64.35) (end 193.4 68.45) (stroke (width 0.05) (type default)) (layer "Edge.Cuts"))
 (gr_line (start 195.2 59.95) (end 201 56.65) (stroke (width 0.05) (type default)) (layer "Edge.Cuts"))
 (gr_line (start 197.2 117.65) (end 198.7 113.15) (stroke (width 0.05) (type default)) (layer "Edge.Cuts"))
 (gr_line (start 197.7 61.25) (end 194.9 64.35) (stroke (width 0.05) (type default)) (layer "Edge.Cuts"))
 (gr_line (start 197.8 52.55) (end 194.9 54.45) (stroke (width 0.05) (type default)) (layer "Edge.Cuts"))
 (gr_line (start 198.7 113.15) (end 200.5 107.75) (stroke (width 0.05) (type default)) (layer "Edge.Cuts"))
 (gr_line (start 198.8 78.95) (end 202.8 77.55) (stroke (width 0.05) (type default)) (layer "Edge.Cuts"))
 (gr_line (start 199.7 79.95) (end 198.8 78.95) (stroke (width 0.05) (type default)) (layer "Edge.Cuts"))
 (gr_line (start 200.4 50.55) (end 197.8 52.55) (stroke (width 0.05) (type default)) (layer "Edge.Cuts"))
 (gr_line (start 200.5 107.75) (end 202.4 103.55) (stroke (width 0.05) (type default)) (layer "Edge.Cuts"))
 (gr_line (start 200.6 58.05) (end 197.7 61.25) (stroke (width 0.05) (type default)) (layer "Edge.Cuts"))
 (gr_line (start 201 56.65) (end 204.4 53.05) (stroke (width 0.05) (type default)) (layer "Edge.Cuts"))
 (gr_line (start 201.5 48.55) (end 200.4 50.55) (stroke (width 0.05) (type default)) (layer "Edge.Cuts"))
 (gr_line (start 201.9 84.75) (end 199.7 79.95) (stroke (width 0.05) (type default)) (layer "Edge.Cuts"))
 (gr_line (start 202.4 103.55) (end 203.7 98.25) (stroke (width 0.05) (type default)) (layer "Edge.Cuts"))
 (gr_line (start 202.8 45.75) (end 201.5 48.55) (stroke (width 0.05) (type default)) (layer "Edge.Cuts"))
 (gr_line (start 202.8 77.55) (end 207.1 74.35) (stroke (width 0.05) (type default)) (layer "Edge.Cuts"))
 (gr_line (start 203.5 91.55) (end 201.9 84.75) (stroke (width 0.05) (type default)) (layer "Edge.Cuts"))
 (gr_line (start 203.7 98.25) (end 203.5 91.55) (stroke (width 0.05) (type default)) (layer "Edge.Cuts"))
 (gr_line (start 203.8 43.75) (end 202.8 45.75) (stroke (width 0.05) (type default)) (layer "Edge.Cuts"))
 (gr_line (start 204.4 53.05) (end 206.8 49.15) (stroke (width 0.05) (type default)) (layer "Edge.Cuts"))
 (gr_line (start 204.9 41.95) (end 203.8 43.75) (stroke (width 0.05) (type default)) (layer "Edge.Cuts"))
 (gr_line (start 205.8 40.75) (end 204.9 41.95) (stroke (width 0.05) (type default)) (layer "Edge.Cuts"))
 (gr_line (start 206 53.75) (end 200.6 58.05) (stroke (width 0.05) (type default)) (layer "Edge.Cuts"))
 (gr_line (start 206.8 40.65) (end 205.8 40.75) (stroke (width 0.05) (type default)) (layer "Edge.Cuts"))
 (gr_line (start 206.8 49.15) (end 208.2 44.35) (stroke (width 0.05) (type default)) (layer "Edge.Cuts"))
 (gr_line (start 207.1 74.35) (end 210.1 70.95) (stroke (width 0.05) (type default)) (layer "Edge.Cuts"))
 (gr_line (start 207.9 41.45) (end 206.8 40.65) (stroke (width 0.05) (type default)) (layer "Edge.Cuts"))
 (gr_line (start 208.2 44.35) (end 207.9 41.45) (stroke (width 0.05) (type default)) (layer "Edge.Cuts"))
 (gr_line (start 210.1 70.95) (end 212.3 66.45) (stroke (width 0.05) (type default)) (layer "Edge.Cuts"))
 (gr_line (start 210.9 49.15) (end 206 53.75) (stroke (width 0.05) (type default)) (layer "Edge.Cuts"))
 (gr_line (start 211.9 52.25) (end 210.9 49.15) (stroke (width 0.05) (type default)) (layer "Edge.Cuts"))
 (gr_line (start 212.3 66.45) (end 213.3 60.55) (stroke (width 0.05) (type default)) (layer "Edge.Cuts"))
 (gr_line (start 212.8 55.75) (end 211.9 52.25) (stroke (width 0.05) (type default)) (layer "Edge.Cuts"))
 (gr_line (start 213.3 60.55) (end 212.8 55.75) (stroke (width 0.05) (type default)) (layer "Edge.Cuts"))
 (segment (start 150.19 105.7) (end 150.19 107.7) (width 0.2) (layer "F.Cu") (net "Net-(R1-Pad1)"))
 (segment (start 150.25 67.25) (end 153.9 70.9) (width 0.2) (layer "F.Cu") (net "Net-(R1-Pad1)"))
 (segment (start 153.9 70.9) (end 153.9 73.598528) (width 0.2) (layer "F.Cu") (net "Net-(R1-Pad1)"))
 (segment (start 153.9 73.598528) (end 155.701472 75.4) (width 0.2) (layer "F.Cu") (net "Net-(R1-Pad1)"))
 (segment (start 151.55 68.55) (end 150.25 67.25) (width 0.2) (layer "F.Cu") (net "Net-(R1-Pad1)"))
 (segment (start 151.55 104.34) (end 151.55 68.55) (width 0.2) (layer "F.Cu") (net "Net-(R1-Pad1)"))
 (segment (start 150.19 105.7) (end 151.55 104.34) (width 0.2) (layer "F.Cu") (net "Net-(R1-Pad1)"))
 (segment (start 150.19 107.7) (end 151.69 109.2) (width 0.2) (layer "F.Cu") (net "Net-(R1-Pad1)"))
 (segment (start 150.25 67.25) (end 143.75 67.25) (width 0.2) (layer "F.Cu") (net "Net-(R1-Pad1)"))
 (segment (start 155.701472 75.4) (end 192.89 75.4) (width 0.2) (layer "F.Cu") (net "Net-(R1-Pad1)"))
 (segment (start 193.14 112.4) (end 194.19 113.45) (width 0.2) (layer "F.Cu") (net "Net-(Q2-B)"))
 (segment (start 187.48 111.084925) (end 188.795075 112.4) (width 0.2) (layer "F.Cu") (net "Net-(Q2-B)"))
 (segment (start 155.9 107.61) (end 157.81 105.7) (width 0.2) (layer "F.Cu") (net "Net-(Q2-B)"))
 (segment (start 187.48 110.215075) (end 187.48 111.084925) (width 0.2) (layer "F.Cu") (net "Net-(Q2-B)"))
 (segment (start 155.9 113.8) (end 155.9 107.61) (width 0.2) (layer "F.Cu") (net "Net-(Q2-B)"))
 (segment (start 182.964925 105.7) (end 187.48 110.215075) (width 0.2) (layer "F.Cu") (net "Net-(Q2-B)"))
 (segment (start 188.795075 112.4) (end 193.14 112.4) (width 0.2) (layer "F.Cu") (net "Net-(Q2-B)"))
 (segment (start 157.81 105.7) (end 182.964925 105.7) (width 0.2) (layer "F.Cu") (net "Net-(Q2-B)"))
 (segment (start 173.5 110.7) (end 170.34 110.7) (width 0.2) (layer "F.Cu") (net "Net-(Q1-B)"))
 (segment (start 173.5 116.69) (end 175.01 118.2) (width 0.2) (layer "F.Cu") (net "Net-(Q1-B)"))
 (segment (start 173.5 110.7) (end 173.5 116.69) (width 0.2) (layer "F.Cu") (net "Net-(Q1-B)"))
 (segment (start 170.34 110.7) (end 167.19 107.55) (width 0.2) (layer "F.Cu") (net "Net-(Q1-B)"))
 (segment (start 178.55 110.65) (end 178.5 110.7) (width 0.2) (layer "F.Cu") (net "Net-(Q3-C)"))
 (segment (start 183.45 110.65) (end 178.55 110.65) (width 0.2) (layer "F.Cu") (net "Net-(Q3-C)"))
 (segment (start 178.5 123.61) (end 175.61 126.5) (width 0.2) (layer "B.Cu") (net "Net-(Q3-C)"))
 (segment (start 178.5 110.7) (end 178.5 123.61) (width 0.2) (layer "B.Cu") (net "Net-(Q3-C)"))
 (segment (start 166.025 88.4) (end 164.825 87.2) (width 0.2) (layer "F.Cu") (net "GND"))
 (segment (start 191.865 79.5) (end 188.625 79.5) (width 0.2) (layer "F.Cu") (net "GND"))
 (segment (start 172.425 94.8) (end 164.825 87.2) (width 0.2) (layer "F.Cu") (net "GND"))
 (segment (start 205.2 66.765) (end 205.2 66.7) (width 0.2) (layer "F.Cu") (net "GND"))
 (segment (start 204.9 66.465) (end 191.865 79.5) (width 0.2) (layer "F.Cu") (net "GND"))
 (segment (start 181.125 87) (end 179.725 88.4) (width 0.2) (layer "F.Cu") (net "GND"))
 (segment (start 172.425 97.2) (end 172.425 94.8) (width 0.2) (layer "F.Cu") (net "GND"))
 (segment (start 204.9 66.465) (end 205.2 66.765) (width 0.2) (layer "F.Cu") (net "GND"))
 (segment (start 205.2 66.7) (end 205.3 66.6) (width 0.2) (layer "F.Cu") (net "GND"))
 (segment (start 179.725 88.4) (end 166.025 88.4) (width 0.2) (layer "F.Cu") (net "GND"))
 (segment (start 188.625 79.5) (end 181.125 87) (width 0.2) (layer "F.Cu") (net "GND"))
 (segment (start 183.665 100.385) (end 196.73 113.45) (width 0.2) (layer "F.Cu") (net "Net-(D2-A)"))
 (segment (start 183.665 87) (end 183.665 100.385) (width 0.2) (layer "F.Cu") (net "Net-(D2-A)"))
 (segment (start 188.53 110.65) (end 175.08 97.2) (width 0.2) (layer "F.Cu") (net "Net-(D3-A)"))
 (segment (start 175.08 97.2) (end 174.965 97.2) (width 0.2) (layer "F.Cu") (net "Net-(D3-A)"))
 (segment (start 172.39 130.9) (end 172.39 131.6) (width 0.2) (layer "F.Cu") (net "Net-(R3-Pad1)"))
 (segment (start 150.25 71.75) (end 143.75 71.75) (width 0.2) (layer "F.Cu") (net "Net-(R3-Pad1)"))
 (segment (start 167.99 126.5) (end 172.39 130.9) (width 0.2) (layer "F.Cu") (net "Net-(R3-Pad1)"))
 (segment (start 162.89 122.7) (end 157.29 122.7) (width 0.2) (layer "B.Cu") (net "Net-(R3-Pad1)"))
 (segment (start 150.25 71.75) (end 150.25 95.25) (width 0.2) (layer "B.Cu") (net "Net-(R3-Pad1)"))
 (segment (start 167.39 118.2) (end 162.89 122.7) (width 0.2) (layer "B.Cu") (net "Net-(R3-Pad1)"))
 (segment (start 167.39 112.39) (end 167.39 118.2) (width 0.2) (layer "B.Cu") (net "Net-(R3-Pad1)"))
 (segment (start 161.09 126.5) (end 167.99 126.5) (width 0.2) (layer "B.Cu") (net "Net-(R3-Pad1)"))
 (segment (start 150.25 95.25) (end 167.39 112.39) (width 0.2) (layer "B.Cu") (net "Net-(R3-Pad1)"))
 (segment (start 157.29 122.7) (end 161.09 126.5) (width 0.2) (layer "B.Cu") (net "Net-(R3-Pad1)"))
 (segment (start 184 122.7) (end 164.91 122.7) (width 0.2) (layer "F.Cu") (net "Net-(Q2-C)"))
 (segment (start 191.65 113.45) (end 191.65 115.05) (width 0.2) (layer "F.Cu") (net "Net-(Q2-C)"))
 (segment (start 189.3 117.4) (end 184 122.7) (width 0.2) (layer "F.Cu") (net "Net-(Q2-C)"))
 (segment (start 191.65 115.05) (end 189.3 117.4) (width 0.2) (layer "F.Cu") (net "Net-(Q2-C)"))
 (segment (start 185.99 110.65) (end 185.99 115.71) (width 0.2) (layer "F.Cu") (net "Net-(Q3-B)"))
 (segment (start 185.99 115.71) (end 184.3 117.4) (width 0.2) (layer "F.Cu") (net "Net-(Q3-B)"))
 (segment (start 180.01 121.69) (end 184.3 117.4) (width 0.2) (layer "B.Cu") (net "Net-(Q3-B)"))
 (segment (start 180.01 131.6) (end 180.01 121.69) (width 0.2) (layer "B.Cu") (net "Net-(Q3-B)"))
 (segment (start 159.31 109.2) (end 159.31 112.21) (width 0.2) (layer "F.Cu") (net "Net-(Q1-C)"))
 (segment (start 164.65 107.55) (end 160.96 107.55) (width 0.2) (layer "F.Cu") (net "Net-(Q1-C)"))
 (segment (start 159.31 112.21) (end 160.9 113.8) (width 0.2) (layer "F.Cu") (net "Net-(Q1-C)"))
 (segment (start 160.96 107.55) (end 159.31 109.2) (width 0.2) (layer "F.Cu") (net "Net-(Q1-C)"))
 (segment (start 167.365 87.2) (end 169.73 89.565) (width 0.2) (layer "B.Cu") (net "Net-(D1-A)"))
 (segment (start 169.73 89.565) (end 169.73 107.55) (width 0.2) (layer "B.Cu") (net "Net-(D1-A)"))
 (segment (start 206.05 69.86) (end 200.51 75.4) (width 0.2) (layer "F.Cu") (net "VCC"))
 (segment (start 204.9 63.925) (end 206.05 65.075) (width 0.2) (layer "F.Cu") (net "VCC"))
 (segment (start 206.05 65.075) (end 206.05 69.86) (width 0.2) (layer "F.Cu") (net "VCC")))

